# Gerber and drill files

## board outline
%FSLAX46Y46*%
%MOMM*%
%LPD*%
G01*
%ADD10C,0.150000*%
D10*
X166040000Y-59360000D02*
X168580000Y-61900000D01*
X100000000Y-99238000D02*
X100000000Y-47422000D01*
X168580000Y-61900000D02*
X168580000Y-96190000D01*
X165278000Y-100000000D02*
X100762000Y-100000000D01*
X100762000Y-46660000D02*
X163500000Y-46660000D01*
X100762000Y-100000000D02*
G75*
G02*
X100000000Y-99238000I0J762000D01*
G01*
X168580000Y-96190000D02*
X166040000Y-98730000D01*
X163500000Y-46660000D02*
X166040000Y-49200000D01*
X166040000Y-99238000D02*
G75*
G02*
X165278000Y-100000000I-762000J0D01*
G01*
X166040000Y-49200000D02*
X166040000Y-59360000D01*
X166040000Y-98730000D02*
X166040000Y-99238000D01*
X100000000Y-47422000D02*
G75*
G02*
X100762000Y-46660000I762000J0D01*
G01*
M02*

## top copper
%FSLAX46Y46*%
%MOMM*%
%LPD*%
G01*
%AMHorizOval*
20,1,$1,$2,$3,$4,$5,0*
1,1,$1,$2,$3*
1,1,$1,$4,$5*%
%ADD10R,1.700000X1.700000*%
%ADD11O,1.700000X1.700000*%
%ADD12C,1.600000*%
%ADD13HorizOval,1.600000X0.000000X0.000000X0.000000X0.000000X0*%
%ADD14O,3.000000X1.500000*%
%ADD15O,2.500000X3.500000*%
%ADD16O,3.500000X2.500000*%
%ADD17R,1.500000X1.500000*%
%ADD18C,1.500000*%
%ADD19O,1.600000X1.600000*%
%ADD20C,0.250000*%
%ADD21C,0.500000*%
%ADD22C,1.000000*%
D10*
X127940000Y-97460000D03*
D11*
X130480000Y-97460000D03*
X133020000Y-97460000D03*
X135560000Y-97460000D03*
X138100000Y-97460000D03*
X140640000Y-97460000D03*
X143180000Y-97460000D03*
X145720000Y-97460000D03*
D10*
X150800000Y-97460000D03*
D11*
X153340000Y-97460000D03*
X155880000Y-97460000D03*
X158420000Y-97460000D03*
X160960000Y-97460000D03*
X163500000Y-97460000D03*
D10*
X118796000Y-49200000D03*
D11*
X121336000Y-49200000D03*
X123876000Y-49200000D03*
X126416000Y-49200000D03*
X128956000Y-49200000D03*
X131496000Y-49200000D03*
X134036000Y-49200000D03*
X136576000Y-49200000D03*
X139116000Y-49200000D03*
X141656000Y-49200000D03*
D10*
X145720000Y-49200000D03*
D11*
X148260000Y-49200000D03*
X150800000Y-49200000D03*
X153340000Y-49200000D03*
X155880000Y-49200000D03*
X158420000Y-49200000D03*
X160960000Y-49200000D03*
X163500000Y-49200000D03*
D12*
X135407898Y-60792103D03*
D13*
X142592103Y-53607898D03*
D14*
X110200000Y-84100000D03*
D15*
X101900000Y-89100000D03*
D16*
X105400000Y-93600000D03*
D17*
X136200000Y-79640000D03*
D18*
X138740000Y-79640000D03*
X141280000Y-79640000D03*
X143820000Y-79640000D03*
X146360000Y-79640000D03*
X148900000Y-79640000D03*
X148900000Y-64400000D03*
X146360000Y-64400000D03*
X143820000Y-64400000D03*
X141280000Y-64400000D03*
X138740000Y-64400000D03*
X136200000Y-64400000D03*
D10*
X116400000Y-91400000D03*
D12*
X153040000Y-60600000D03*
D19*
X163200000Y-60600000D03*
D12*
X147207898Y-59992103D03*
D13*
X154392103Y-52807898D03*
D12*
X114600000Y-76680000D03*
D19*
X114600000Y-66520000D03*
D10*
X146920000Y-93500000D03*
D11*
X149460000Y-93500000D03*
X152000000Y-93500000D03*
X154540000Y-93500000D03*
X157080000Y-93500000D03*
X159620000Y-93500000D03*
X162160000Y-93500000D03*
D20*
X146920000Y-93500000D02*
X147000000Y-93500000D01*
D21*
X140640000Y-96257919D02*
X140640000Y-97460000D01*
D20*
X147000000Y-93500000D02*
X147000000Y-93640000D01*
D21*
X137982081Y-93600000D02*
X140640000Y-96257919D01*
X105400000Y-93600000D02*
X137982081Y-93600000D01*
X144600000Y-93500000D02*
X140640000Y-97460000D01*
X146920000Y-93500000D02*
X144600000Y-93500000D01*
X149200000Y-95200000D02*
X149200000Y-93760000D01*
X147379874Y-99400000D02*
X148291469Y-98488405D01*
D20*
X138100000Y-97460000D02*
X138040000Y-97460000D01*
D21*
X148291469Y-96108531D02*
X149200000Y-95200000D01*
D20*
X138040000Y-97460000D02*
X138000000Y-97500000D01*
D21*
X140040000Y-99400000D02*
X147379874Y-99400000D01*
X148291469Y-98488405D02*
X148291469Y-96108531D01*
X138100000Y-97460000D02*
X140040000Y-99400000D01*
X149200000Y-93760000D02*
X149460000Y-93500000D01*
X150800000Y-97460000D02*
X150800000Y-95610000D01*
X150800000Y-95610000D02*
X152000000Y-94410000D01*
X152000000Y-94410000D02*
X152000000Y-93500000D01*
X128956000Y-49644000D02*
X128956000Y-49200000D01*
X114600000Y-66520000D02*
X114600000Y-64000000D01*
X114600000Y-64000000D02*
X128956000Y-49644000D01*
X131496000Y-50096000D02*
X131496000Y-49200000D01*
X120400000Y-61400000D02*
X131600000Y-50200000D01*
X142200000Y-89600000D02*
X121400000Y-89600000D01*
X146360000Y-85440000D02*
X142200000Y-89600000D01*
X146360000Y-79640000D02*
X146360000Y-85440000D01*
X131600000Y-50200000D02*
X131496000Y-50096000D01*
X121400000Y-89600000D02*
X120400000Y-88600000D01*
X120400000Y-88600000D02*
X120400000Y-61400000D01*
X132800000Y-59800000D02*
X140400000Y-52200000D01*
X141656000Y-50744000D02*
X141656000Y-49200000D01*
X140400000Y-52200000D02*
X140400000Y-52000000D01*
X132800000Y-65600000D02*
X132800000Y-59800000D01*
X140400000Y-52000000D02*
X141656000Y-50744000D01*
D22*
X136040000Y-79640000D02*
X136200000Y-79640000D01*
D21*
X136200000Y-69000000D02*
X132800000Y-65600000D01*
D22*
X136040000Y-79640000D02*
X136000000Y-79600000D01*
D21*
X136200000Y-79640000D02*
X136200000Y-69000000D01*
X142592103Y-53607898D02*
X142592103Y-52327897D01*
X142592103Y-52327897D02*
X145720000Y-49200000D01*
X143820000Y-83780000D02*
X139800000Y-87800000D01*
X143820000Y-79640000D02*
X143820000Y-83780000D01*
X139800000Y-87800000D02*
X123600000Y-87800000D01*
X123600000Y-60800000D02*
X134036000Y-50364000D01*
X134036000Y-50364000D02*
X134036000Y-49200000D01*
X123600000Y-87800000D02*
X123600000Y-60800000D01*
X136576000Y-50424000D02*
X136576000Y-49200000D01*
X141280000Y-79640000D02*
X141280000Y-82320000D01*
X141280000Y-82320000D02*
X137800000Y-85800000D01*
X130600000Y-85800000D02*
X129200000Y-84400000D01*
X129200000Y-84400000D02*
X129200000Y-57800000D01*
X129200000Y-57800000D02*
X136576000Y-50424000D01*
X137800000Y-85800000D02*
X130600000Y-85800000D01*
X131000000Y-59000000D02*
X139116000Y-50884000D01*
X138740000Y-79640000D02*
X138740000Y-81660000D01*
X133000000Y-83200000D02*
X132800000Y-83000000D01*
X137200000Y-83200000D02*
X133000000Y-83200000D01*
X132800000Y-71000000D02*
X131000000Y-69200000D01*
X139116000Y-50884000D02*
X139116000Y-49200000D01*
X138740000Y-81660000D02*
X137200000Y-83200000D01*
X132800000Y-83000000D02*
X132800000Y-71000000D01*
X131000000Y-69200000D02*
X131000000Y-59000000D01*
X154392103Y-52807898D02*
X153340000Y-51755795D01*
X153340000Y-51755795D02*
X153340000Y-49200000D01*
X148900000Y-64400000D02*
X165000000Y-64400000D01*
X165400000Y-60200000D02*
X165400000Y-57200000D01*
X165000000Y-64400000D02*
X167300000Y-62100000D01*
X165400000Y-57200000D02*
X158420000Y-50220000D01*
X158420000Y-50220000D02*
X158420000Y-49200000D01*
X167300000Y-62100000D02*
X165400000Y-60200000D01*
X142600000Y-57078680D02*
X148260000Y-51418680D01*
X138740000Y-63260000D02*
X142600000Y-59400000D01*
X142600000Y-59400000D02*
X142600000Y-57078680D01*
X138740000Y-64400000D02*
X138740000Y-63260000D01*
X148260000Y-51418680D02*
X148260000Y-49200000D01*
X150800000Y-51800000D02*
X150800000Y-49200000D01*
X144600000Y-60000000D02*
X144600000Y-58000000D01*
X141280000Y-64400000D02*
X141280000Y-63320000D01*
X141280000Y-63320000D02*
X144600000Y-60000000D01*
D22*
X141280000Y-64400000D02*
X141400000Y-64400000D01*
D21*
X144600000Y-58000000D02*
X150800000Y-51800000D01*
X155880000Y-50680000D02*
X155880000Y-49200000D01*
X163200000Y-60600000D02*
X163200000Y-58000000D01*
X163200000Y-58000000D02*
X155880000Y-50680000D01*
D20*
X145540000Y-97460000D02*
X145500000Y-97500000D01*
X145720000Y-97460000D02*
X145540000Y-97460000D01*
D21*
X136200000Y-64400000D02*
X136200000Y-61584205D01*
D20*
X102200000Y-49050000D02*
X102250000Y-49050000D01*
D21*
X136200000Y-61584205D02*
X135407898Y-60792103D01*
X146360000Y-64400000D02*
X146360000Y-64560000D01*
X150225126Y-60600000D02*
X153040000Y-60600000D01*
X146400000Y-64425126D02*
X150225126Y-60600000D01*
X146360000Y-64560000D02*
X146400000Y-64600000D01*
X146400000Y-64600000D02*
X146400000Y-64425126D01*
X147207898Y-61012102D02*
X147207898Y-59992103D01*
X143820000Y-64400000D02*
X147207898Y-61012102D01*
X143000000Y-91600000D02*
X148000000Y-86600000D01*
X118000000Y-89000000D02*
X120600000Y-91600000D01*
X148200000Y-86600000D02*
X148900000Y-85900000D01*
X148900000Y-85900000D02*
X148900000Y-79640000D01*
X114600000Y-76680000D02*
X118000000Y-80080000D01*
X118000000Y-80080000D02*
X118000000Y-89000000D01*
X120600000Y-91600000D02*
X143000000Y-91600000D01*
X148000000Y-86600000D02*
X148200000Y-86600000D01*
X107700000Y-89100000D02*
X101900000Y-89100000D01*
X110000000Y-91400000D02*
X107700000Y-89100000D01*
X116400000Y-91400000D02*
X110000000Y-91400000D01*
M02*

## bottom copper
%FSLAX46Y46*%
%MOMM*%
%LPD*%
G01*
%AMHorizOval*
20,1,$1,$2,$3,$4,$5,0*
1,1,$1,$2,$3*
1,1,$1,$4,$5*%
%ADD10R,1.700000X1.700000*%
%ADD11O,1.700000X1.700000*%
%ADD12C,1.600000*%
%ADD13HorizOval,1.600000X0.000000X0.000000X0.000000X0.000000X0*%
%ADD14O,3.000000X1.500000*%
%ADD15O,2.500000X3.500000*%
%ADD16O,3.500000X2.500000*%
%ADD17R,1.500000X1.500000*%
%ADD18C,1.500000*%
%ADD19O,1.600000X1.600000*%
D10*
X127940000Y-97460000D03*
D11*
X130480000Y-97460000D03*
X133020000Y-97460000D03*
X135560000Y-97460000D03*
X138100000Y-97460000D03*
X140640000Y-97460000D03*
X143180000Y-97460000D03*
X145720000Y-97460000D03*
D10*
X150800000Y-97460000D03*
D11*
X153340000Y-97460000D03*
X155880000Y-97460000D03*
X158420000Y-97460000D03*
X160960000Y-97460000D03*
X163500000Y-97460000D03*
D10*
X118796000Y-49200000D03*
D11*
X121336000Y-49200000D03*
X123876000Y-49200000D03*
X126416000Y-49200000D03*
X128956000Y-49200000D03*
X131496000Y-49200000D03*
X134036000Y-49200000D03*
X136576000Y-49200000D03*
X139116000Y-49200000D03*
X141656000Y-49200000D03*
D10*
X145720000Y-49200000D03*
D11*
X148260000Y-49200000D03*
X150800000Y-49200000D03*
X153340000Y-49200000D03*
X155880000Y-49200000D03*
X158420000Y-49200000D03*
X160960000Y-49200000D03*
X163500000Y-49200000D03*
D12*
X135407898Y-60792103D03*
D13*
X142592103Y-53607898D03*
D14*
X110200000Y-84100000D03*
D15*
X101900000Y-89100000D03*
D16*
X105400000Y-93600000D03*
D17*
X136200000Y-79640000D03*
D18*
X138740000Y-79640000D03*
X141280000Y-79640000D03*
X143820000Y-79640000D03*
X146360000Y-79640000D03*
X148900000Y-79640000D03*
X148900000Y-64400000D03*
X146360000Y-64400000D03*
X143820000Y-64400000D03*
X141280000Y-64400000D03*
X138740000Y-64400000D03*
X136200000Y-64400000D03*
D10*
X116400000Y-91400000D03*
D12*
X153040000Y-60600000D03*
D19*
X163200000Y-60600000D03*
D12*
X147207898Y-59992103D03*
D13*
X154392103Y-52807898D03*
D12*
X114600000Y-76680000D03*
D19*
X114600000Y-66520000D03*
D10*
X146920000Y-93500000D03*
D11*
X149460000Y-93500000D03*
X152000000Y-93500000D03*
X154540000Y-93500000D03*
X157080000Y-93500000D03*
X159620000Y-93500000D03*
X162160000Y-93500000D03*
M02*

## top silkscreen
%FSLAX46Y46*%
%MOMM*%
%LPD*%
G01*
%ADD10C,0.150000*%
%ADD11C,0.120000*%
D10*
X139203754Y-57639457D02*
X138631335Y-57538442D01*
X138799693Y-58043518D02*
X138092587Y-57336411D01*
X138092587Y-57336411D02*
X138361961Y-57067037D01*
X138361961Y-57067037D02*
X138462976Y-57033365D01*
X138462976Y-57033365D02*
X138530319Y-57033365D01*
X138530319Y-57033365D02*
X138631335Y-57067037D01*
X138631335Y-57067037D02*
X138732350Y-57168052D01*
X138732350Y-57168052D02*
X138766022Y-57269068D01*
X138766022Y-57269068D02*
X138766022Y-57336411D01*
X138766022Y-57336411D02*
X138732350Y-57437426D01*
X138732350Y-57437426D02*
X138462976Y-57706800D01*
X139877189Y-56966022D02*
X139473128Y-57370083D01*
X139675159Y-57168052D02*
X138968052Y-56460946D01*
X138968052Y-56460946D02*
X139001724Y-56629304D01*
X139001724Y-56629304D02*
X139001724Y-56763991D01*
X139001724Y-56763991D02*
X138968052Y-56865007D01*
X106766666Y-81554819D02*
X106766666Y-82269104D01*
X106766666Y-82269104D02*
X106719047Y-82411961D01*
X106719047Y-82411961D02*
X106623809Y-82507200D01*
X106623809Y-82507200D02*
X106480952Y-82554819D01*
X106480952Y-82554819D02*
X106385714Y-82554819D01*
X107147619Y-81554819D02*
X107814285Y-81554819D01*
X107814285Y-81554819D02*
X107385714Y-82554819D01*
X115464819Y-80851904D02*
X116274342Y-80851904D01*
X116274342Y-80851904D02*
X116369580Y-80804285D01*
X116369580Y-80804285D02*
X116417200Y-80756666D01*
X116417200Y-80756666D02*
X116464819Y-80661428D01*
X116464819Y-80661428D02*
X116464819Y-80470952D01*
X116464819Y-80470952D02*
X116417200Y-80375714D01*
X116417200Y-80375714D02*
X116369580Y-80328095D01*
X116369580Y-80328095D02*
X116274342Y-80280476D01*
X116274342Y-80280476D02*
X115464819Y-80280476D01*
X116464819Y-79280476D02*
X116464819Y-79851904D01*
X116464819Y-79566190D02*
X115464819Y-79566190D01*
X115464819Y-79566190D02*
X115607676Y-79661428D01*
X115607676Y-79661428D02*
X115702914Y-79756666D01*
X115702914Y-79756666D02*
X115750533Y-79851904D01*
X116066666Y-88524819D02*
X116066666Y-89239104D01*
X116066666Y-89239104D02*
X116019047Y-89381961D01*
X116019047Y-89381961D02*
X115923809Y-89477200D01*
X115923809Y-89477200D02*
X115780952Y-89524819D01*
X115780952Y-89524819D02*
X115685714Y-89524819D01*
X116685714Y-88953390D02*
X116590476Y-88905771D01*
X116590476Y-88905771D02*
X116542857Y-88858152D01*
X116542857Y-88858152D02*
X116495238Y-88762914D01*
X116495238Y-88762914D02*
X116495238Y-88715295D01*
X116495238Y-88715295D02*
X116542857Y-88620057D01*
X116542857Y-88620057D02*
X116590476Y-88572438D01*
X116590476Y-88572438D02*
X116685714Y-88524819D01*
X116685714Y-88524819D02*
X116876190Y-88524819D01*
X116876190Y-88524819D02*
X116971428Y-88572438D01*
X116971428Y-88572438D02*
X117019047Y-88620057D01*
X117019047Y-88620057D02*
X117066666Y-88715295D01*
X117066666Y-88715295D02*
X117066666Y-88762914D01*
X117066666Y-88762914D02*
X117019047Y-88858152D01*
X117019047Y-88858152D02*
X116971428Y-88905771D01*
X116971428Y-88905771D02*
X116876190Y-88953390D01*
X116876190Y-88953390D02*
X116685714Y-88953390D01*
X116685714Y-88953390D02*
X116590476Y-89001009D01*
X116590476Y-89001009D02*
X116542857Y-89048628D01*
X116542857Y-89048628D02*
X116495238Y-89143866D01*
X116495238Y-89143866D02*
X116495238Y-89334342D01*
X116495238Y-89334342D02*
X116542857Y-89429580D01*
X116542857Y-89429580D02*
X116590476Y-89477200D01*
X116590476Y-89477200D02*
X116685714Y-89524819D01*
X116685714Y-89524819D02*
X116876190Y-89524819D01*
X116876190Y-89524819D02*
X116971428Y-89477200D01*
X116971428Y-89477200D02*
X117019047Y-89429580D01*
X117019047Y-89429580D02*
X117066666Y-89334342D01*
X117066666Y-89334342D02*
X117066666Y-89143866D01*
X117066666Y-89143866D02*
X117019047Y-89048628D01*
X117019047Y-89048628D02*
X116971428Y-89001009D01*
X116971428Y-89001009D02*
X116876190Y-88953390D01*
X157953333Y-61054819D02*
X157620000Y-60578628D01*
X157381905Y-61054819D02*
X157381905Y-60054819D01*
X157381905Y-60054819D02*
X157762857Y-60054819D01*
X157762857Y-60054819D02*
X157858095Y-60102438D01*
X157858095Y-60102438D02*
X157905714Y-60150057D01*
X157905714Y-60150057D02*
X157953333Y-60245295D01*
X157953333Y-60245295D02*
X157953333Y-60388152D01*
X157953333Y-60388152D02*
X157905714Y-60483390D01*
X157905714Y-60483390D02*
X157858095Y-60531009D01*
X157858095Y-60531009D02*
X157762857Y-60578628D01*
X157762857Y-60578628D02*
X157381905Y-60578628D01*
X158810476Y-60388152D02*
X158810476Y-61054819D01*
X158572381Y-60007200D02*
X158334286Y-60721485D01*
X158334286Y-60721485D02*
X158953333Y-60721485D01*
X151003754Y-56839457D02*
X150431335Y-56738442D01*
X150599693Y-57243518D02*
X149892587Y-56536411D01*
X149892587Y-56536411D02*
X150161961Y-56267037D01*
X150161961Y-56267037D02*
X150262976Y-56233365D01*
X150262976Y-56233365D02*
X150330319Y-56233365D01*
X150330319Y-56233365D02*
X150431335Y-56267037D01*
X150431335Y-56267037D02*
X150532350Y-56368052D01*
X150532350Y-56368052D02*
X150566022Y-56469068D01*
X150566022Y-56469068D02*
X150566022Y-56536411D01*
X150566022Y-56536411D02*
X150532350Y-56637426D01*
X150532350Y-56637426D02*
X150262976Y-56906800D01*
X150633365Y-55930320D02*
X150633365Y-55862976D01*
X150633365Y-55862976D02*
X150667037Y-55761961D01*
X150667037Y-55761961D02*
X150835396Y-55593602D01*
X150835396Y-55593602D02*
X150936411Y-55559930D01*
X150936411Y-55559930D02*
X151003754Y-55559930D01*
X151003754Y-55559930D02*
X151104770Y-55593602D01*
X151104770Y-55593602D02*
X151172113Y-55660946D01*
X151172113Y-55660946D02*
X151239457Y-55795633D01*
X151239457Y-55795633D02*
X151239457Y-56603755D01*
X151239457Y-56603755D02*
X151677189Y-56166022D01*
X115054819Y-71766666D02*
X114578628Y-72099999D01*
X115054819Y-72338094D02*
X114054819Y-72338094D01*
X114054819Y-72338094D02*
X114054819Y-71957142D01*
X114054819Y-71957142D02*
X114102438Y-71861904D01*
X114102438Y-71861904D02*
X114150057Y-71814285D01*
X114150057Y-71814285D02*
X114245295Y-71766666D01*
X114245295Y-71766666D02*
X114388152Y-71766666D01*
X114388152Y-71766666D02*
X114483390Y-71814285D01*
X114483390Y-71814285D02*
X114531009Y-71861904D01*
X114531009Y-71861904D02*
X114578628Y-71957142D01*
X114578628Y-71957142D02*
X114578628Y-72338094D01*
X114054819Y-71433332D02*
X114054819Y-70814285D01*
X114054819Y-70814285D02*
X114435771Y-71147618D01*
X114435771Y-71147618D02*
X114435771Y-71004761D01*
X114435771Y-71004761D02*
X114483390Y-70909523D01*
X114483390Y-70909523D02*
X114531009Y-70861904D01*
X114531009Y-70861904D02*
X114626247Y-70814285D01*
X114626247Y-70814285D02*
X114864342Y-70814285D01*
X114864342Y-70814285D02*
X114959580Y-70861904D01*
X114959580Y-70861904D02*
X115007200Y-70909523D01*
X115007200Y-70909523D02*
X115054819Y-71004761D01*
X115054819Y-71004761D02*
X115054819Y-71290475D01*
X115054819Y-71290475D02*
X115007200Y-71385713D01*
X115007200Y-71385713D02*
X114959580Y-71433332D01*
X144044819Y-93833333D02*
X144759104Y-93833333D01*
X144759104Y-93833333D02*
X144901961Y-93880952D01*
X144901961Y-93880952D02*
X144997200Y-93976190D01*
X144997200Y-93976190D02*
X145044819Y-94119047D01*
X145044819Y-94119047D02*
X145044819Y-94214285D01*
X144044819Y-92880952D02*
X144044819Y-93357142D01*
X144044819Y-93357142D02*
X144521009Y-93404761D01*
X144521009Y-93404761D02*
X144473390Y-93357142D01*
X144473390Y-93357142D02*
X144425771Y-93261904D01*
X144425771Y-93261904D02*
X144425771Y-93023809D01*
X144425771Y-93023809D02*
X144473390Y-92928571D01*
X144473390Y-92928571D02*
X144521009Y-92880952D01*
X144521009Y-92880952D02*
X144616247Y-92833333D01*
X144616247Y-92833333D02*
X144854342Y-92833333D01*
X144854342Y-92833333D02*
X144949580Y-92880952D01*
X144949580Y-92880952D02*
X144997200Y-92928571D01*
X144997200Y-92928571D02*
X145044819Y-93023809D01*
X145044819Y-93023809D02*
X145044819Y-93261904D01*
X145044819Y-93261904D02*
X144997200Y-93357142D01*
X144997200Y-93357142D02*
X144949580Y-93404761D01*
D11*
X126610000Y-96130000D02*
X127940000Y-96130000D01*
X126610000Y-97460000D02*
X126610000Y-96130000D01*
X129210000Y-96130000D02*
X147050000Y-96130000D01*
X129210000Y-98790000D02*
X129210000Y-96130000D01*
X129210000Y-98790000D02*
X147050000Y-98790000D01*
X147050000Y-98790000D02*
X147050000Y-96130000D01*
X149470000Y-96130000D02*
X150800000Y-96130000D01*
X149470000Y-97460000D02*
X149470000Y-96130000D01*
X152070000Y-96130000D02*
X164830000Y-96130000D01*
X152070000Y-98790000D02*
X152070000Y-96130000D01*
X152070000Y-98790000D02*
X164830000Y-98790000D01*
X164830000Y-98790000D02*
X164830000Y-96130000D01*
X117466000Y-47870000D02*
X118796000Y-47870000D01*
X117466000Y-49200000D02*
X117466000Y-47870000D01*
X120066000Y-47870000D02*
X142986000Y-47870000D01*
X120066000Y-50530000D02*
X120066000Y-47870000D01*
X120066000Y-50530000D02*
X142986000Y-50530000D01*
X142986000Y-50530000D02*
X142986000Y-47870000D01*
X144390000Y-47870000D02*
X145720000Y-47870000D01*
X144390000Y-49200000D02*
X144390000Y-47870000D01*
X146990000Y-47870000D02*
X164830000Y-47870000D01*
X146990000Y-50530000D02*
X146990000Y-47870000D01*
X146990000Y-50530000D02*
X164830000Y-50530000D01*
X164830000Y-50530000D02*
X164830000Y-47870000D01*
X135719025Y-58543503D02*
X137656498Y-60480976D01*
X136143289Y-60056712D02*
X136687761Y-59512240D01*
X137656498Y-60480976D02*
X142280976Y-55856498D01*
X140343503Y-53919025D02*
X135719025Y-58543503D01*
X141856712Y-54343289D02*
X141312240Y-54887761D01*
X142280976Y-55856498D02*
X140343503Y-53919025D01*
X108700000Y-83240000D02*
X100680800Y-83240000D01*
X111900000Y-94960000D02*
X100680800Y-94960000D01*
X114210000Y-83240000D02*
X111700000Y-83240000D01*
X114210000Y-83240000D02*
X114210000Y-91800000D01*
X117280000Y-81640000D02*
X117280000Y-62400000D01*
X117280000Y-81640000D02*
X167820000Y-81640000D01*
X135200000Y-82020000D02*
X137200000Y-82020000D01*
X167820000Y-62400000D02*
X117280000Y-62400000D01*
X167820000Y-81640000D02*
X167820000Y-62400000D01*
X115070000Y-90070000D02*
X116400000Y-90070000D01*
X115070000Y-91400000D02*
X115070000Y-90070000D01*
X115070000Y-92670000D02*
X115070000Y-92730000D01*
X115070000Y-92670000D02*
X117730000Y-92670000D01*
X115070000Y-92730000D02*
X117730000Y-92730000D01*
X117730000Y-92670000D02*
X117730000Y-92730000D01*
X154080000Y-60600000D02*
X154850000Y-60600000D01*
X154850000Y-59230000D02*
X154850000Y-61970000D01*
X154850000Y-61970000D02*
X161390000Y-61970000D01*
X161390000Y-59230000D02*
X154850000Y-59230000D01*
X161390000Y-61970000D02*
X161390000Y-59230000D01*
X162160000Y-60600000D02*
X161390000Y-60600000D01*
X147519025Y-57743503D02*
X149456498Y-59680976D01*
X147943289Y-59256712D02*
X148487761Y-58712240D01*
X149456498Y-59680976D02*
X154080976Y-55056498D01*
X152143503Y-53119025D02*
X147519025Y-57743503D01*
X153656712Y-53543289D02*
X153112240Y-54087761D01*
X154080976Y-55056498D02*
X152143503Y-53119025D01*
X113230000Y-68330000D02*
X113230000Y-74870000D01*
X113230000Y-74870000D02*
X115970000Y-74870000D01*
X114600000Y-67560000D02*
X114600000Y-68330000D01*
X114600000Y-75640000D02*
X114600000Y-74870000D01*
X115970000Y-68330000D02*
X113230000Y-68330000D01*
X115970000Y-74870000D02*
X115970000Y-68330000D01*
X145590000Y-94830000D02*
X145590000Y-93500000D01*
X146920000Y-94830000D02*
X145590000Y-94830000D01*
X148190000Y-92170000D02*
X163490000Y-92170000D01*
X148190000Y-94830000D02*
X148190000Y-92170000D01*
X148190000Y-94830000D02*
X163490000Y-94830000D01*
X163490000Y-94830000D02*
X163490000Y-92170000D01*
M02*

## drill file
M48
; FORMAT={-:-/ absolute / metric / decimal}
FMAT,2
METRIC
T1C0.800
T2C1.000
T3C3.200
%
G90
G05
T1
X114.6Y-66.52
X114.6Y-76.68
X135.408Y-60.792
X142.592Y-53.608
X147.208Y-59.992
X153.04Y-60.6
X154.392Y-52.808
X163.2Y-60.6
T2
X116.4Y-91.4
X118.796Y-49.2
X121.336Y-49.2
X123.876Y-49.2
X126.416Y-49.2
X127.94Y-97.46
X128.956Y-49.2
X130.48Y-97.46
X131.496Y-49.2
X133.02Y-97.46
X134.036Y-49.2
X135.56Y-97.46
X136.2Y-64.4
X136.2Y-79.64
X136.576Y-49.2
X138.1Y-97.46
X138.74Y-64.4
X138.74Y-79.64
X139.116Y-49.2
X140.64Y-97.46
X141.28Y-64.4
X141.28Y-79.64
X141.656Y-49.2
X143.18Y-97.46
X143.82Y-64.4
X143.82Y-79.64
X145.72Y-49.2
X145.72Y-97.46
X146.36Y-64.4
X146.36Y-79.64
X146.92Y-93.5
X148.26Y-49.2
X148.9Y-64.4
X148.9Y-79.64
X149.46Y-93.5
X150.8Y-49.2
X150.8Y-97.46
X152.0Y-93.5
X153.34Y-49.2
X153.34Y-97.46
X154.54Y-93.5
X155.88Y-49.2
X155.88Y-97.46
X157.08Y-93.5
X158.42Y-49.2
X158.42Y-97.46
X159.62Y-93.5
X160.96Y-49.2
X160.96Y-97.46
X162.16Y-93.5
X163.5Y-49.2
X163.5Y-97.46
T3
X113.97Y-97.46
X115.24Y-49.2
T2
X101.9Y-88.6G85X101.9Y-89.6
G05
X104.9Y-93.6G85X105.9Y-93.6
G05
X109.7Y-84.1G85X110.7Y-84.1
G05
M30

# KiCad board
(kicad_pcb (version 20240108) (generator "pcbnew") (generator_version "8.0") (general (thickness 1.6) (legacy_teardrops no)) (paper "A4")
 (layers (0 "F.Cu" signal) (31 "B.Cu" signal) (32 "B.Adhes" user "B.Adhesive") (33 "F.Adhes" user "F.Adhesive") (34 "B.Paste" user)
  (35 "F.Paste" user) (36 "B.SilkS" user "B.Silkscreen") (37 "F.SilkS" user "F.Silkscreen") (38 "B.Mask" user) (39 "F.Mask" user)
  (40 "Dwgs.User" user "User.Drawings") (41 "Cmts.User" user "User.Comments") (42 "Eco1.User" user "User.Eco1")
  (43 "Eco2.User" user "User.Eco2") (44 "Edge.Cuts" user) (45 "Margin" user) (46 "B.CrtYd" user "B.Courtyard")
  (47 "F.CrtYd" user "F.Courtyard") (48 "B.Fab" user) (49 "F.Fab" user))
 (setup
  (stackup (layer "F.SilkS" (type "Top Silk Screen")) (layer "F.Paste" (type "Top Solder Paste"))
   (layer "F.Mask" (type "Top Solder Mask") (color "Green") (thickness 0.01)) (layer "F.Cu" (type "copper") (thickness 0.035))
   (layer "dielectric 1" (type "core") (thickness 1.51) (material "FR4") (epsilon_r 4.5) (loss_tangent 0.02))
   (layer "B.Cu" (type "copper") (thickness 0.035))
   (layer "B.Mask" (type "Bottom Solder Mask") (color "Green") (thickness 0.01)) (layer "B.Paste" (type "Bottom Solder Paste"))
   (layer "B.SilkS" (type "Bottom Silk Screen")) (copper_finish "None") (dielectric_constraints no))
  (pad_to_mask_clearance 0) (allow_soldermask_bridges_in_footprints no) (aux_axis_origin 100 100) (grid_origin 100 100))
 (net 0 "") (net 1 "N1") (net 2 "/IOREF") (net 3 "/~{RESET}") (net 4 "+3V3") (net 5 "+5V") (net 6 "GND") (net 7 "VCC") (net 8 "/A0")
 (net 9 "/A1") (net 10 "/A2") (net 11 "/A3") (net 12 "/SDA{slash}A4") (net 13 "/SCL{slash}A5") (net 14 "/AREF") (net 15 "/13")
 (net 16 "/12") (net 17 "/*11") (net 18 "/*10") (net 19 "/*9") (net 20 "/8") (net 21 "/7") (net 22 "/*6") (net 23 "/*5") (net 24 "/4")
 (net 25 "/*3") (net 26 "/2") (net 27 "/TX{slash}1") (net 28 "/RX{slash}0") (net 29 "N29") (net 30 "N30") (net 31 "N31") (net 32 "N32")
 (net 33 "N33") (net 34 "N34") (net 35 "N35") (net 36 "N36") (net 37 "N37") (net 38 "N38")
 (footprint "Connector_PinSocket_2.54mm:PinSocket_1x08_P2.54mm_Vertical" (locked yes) (layer "F.Cu") (at 127.94 97.46 90)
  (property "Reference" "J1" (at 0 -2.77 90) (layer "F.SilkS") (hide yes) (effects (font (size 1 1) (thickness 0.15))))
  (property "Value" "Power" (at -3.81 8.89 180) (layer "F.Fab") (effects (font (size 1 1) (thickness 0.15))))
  (fp_line (start 1.33 -1.33) (end 1.33 0) (stroke (width 0.12) (type solid)) (layer "F.SilkS"))
  (fp_line (start 0 -1.33) (end 1.33 -1.33) (stroke (width 0.12) (type solid)) (layer "F.SilkS"))
  (fp_line (start 1.33 1.27) (end 1.33 19.11) (stroke (width 0.12) (type solid)) (layer "F.SilkS"))
  (fp_line (start -1.33 1.27) (end 1.33 1.27) (stroke (width 0.12) (type solid)) (layer "F.SilkS"))
  (fp_line (start -1.33 1.27) (end -1.33 19.11) (stroke (width 0.12) (type solid)) (layer "F.SilkS"))
  (fp_line (start -1.33 19.11) (end 1.33 19.11) (stroke (width 0.12) (type solid)) (layer "F.SilkS"))
  (pad "1" thru_hole rect (at 0 0 90) (size 1.7 1.7) (drill 1) (layers "*.Cu" "*.Mask") (remove_unused_layers no) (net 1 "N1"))
  (pad "2" thru_hole oval (at 0 2.54 90) (size 1.7 1.7) (drill 1) (layers "*.Cu" "*.Mask") (remove_unused_layers no) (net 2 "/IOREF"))
  (pad "3" thru_hole oval (at 0 5.08 90) (size 1.7 1.7) (drill 1) (layers "*.Cu" "*.Mask") (remove_unused_layers no) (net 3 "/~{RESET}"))
  (pad "4" thru_hole oval (at 0 7.62 90) (size 1.7 1.7) (drill 1) (layers "*.Cu" "*.Mask") (remove_unused_layers no) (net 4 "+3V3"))
  (pad "5" thru_hole oval (at 0 10.16 90) (size 1.7 1.7) (drill 1) (layers "*.Cu" "*.Mask") (remove_unused_layers no) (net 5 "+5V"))
  (pad "6" thru_hole oval (at 0 12.7 90) (size 1.7 1.7) (drill 1) (layers "*.Cu" "*.Mask") (remove_unused_layers no) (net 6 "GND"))
  (pad "7" thru_hole oval (at 0 15.24 90) (size 1.7 1.7) (drill 1) (layers "*.Cu" "*.Mask") (remove_unused_layers no) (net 6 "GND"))
  (pad "8" thru_hole oval (at 0 17.78 90) (size 1.7 1.7) (drill 1) (layers "*.Cu" "*.Mask") (remove_unused_layers no) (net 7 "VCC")))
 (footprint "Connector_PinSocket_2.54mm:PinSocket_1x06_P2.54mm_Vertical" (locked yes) (layer "F.Cu") (at 150.8 97.46 90)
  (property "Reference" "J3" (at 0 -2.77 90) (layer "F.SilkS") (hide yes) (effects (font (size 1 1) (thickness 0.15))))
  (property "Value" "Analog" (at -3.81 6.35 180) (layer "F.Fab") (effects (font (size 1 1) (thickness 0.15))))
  (fp_line (start 1.33 -1.33) (end 1.33 0) (stroke (width 0.12) (type solid)) (layer "F.SilkS"))
  (fp_line (start 0 -1.33) (end 1.33 -1.33) (stroke (width 0.12) (type solid)) (layer "F.SilkS"))
  (fp_line (start 1.33 1.27) (end 1.33 14.03) (stroke (width 0.12) (type solid)) (layer "F.SilkS"))
  (fp_line (start -1.33 1.27) (end 1.33 1.27) (stroke (width 0.12) (type solid)) (layer "F.SilkS"))
  (fp_line (start -1.33 1.27) (end -1.33 14.03) (stroke (width 0.12) (type solid)) (layer "F.SilkS"))
  (fp_line (start -1.33 14.03) (end 1.33 14.03) (stroke (width 0.12) (type solid)) (layer "F.SilkS"))
  (pad "1" thru_hole rect (at 0 0 90) (size 1.7 1.7) (drill 1) (layers "*.Cu" "*.Mask") (remove_unused_layers no) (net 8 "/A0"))
  (pad "2" thru_hole oval (at 0 2.54 90) (size 1.7 1.7) (drill 1) (layers "*.Cu" "*.Mask") (remove_unused_layers no) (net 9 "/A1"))
  (pad "3" thru_hole oval (at 0 5.08 90) (size 1.7 1.7) (drill 1) (layers "*.Cu" "*.Mask") (remove_unused_layers no) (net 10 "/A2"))
  (pad "4" thru_hole oval (at 0 7.62 90) (size 1.7 1.7) (drill 1) (layers "*.Cu" "*.Mask") (remove_unused_layers no) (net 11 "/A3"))
  (pad "5" thru_hole oval (at 0 10.16 90) (size 1.7 1.7) (drill 1) (layers "*.Cu" "*.Mask") (remove_unused_layers no)
   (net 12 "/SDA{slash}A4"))
  (pad "6" thru_hole oval (at 0 12.7 90) (size 1.7 1.7) (drill 1) (layers "*.Cu" "*.Mask") (remove_unused_layers no)
   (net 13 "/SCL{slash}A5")))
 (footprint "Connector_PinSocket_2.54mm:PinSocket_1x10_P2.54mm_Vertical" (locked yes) (layer "F.Cu") (at 118.796 49.2 90)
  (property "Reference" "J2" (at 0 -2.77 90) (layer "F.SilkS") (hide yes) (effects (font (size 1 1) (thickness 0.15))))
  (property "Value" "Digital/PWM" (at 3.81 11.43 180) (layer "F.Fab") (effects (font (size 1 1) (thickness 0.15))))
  (fp_line (start 1.33 -1.33) (end 1.33 0) (stroke (width 0.12) (type solid)) (layer "F.SilkS"))
  (fp_line (start 0 -1.33) (end 1.33 -1.33) (stroke (width 0.12) (type solid)) (layer "F.SilkS"))
  (fp_line (start 1.33 1.27) (end 1.33 24.19) (stroke (width 0.12) (type solid)) (layer "F.SilkS"))
  (fp_line (start -1.33 1.27) (end 1.33 1.27) (stroke (width 0.12) (type solid)) (layer "F.SilkS"))
  (fp_line (start -1.33 1.27) (end -1.33 24.19) (stroke (width 0.12) (type solid)) (layer "F.SilkS"))
  (fp_line (start -1.33 24.19) (end 1.33 24.19) (stroke (width 0.12) (type solid)) (layer "F.SilkS"))
  (pad "1" thru_hole rect (at 0 0 90) (size 1.7 1.7) (drill 1) (layers "*.Cu" "*.Mask") (remove_unused_layers no) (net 13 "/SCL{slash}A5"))
  (pad "2" thru_hole oval (at 0 2.54 90) (size 1.7 1.7) (drill 1) (layers "*.Cu" "*.Mask") (remove_unused_layers no)
   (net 12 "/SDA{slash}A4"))
  (pad "3" thru_hole oval (at 0 5.08 90) (size 1.7 1.7) (drill 1) (layers "*.Cu" "*.Mask") (remove_unused_layers no) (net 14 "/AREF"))
  (pad "4" thru_hole oval (at 0 7.62 90) (size 1.7 1.7) (drill 1) (layers "*.Cu" "*.Mask") (remove_unused_layers no) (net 6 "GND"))
  (pad "5" thru_hole oval (at 0 10.16 90) (size 1.7 1.7) (drill 1) (layers "*.Cu" "*.Mask") (remove_unused_layers no) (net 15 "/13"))
  (pad "6" thru_hole oval (at 0 12.7 90) (size 1.7 1.7) (drill 1) (layers "*.Cu" "*.Mask") (remove_unused_layers no) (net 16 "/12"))
  (pad "7" thru_hole oval (at 0 15.24 90) (size 1.7 1.7) (drill 1) (layers "*.Cu" "*.Mask") (remove_unused_layers no) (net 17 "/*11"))
  (pad "8" thru_hole oval (at 0 17.78 90) (size 1.7 1.7) (drill 1) (layers "*.Cu" "*.Mask") (remove_unused_layers no) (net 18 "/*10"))
  (pad "9" thru_hole oval (at 0 20.32 90) (size 1.7 1.7) (drill 1) (layers "*.Cu" "*.Mask") (remove_unused_layers no) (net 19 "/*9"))
  (pad "10" thru_hole oval (at 0 22.86 90) (size 1.7 1.7) (drill 1) (layers "*.Cu" "*.Mask") (remove_unused_layers no) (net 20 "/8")))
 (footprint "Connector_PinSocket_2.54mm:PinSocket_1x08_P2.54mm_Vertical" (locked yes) (layer "F.Cu") (at 145.72 49.2 90)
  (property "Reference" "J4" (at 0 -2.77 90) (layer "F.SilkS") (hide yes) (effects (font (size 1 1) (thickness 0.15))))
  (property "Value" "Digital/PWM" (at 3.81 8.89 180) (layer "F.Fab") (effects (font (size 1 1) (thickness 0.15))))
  (fp_line (start 1.33 -1.33) (end 1.33 0) (stroke (width 0.12) (type solid)) (layer "F.SilkS"))
  (fp_line (start 0 -1.33) (end 1.33 -1.33) (stroke (width 0.12) (type solid)) (layer "F.SilkS"))
  (fp_line (start 1.33 1.27) (end 1.33 19.11) (stroke (width 0.12) (type solid)) (layer "F.SilkS"))
  (fp_line (start -1.33 1.27) (end 1.33 1.27) (stroke (width 0.12) (type solid)) (layer "F.SilkS"))
  (fp_line (start -1.33 1.27) (end -1.33 19.11) (stroke (width 0.12) (type solid)) (layer "F.SilkS"))
  (fp_line (start -1.33 19.11) (end 1.33 19.11) (stroke (width 0.12) (type solid)) (layer "F.SilkS"))
  (pad "1" thru_hole rect (at 0 0 90) (size 1.7 1.7) (drill 1) (layers "*.Cu" "*.Mask") (remove_unused_layers no) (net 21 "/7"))
  (pad "2" thru_hole oval (at 0 2.54 90) (size 1.7 1.7) (drill 1) (layers "*.Cu" "*.Mask") (remove_unused_layers no) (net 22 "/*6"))
  (pad "3" thru_hole oval (at 0 5.08 90) (size 1.7 1.7) (drill 1) (layers "*.Cu" "*.Mask") (remove_unused_layers no) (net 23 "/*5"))
  (pad "4" thru_hole oval (at 0 7.62 90) (size 1.7 1.7) (drill 1) (layers "*.Cu" "*.Mask") (remove_unused_layers no) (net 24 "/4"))
  (pad "5" thru_hole oval (at 0 10.16 90) (size 1.7 1.7) (drill 1) (layers "*.Cu" "*.Mask") (remove_unused_layers no) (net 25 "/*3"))
  (pad "6" thru_hole oval (at 0 12.7 90) (size 1.7 1.7) (drill 1) (layers "*.Cu" "*.Mask") (remove_unused_layers no) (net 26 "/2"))
  (pad "7" thru_hole oval (at 0 15.24 90) (size 1.7 1.7) (drill 1) (layers "*.Cu" "*.Mask") (remove_unused_layers no) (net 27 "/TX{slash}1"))
  (pad "8" thru_hole oval (at 0 17.78 90) (size 1.7 1.7) (drill 1) (layers "*.Cu" "*.Mask") (remove_unused_layers no) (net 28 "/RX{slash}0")))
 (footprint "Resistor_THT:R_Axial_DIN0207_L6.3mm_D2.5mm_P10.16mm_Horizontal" (layer "F.Cu") (at 135.407898 60.792103 45)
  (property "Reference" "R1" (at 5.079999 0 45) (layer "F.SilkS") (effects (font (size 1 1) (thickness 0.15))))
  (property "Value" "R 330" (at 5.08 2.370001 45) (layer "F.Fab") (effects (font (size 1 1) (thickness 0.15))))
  (fp_line (start 1.81 -1.37) (end 1.81 1.37) (stroke (width 0.12) (type solid)) (layer "F.SilkS"))
  (fp_line (start 1.04 0) (end 1.81 0) (stroke (width 0.12) (type solid)) (layer "F.SilkS"))
  (fp_line (start 1.81 1.37) (end 8.35 1.37) (stroke (width 0.12) (type solid)) (layer "F.SilkS"))
  (fp_line (start 8.35 -1.37) (end 1.81 -1.37) (stroke (width 0.12) (type solid)) (layer "F.SilkS"))
  (fp_line (start 9.12 0) (end 8.350001 0) (stroke (width 0.12) (type solid)) (layer "F.SilkS"))
  (fp_line (start 8.35 1.37) (end 8.35 -1.37) (stroke (width 0.12) (type solid)) (layer "F.SilkS"))
  (pad "1" thru_hole circle (at 0 0 45) (size 1.6 1.6) (drill 0.8) (layers "*.Cu" "*.Mask") (remove_unused_layers no) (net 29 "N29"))
  (pad "2" thru_hole oval (at 10.16 0 45) (size 1.6 1.6) (drill 0.8) (layers "*.Cu" "*.Mask") (remove_unused_layers no) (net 21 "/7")))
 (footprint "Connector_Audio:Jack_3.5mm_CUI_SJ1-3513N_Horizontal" (layer "F.Cu") (at 101.9 89.1)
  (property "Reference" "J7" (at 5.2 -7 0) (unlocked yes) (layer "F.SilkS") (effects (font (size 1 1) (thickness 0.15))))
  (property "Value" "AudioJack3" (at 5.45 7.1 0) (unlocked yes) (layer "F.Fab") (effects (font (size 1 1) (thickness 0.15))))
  (fp_line (start 6.8 -5.86) (end -1.2192 -5.86) (stroke (width 0.12) (type solid)) (layer "F.SilkS"))
  (fp_line (start 10 5.86) (end -1.2192 5.86) (stroke (width 0.12) (type solid)) (layer "F.SilkS"))
  (fp_line (start 12.31 -5.86) (end 9.8 -5.86) (stroke (width 0.12) (type solid)) (layer "F.SilkS"))
  (fp_line (start 12.31 -5.86) (end 12.31 2.7) (stroke (width 0.12) (type solid)) (layer "F.SilkS"))
  (pad "R" thru_hole oval (at 8.3 -5) (size 3 1.5) (drill oval 2 1) (layers "*.Cu" "*.Mask") (remove_unused_layers no) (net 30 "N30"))
  (pad "S" thru_hole oval (at 0 0 270) (size 3.5 2.5) (drill oval 2 1) (layers "*.Cu" "*.Mask") (remove_unused_layers no) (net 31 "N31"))
  (pad "T" thru_hole oval (at 3.5 4.5) (size 3.5 2.5) (drill oval 2 1) (layers "*.Cu" "*.Mask") (remove_unused_layers no) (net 6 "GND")))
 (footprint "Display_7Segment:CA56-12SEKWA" (layer "F.Cu") (at 136.2 79.64 90)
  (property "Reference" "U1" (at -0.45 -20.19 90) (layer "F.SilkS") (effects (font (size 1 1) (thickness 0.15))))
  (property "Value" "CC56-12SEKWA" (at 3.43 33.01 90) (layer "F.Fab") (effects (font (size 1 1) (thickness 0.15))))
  (fp_line (start -2 -18.92) (end 17.24 -18.92) (stroke (width 0.12) (type solid)) (layer "F.SilkS"))
  (fp_line (start -2 -18.92) (end -2 31.62) (stroke (width 0.12) (type solid)) (layer "F.SilkS"))
  (fp_line (start -2.38 -1) (end -2.38 1) (stroke (width 0.12) (type solid)) (layer "F.SilkS"))
  (fp_line (start 17.24 31.62) (end 17.24 -18.92) (stroke (width 0.12) (type solid)) (layer "F.SilkS"))
  (fp_line (start -2 31.62) (end 17.24 31.62) (stroke (width 0.12) (type solid)) (layer "F.SilkS"))
  (pad "1" thru_hole rect (at 0 0 90) (size 1.5 1.5) (drill 1) (layers "*.Cu" "*.Mask") (remove_unused_layers no) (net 20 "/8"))
  (pad "2" thru_hole circle (at 0 2.54 90) (size 1.5 1.5) (drill 1) (layers "*.Cu" "*.Mask") (remove_unused_layers no) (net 19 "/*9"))
  (pad "3" thru_hole circle (at 0 5.08 90) (size 1.5 1.5) (drill 1) (layers "*.Cu" "*.Mask") (remove_unused_layers no) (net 18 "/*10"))
  (pad "4" thru_hole circle (at 0 7.62 90) (size 1.5 1.5) (drill 1) (layers "*.Cu" "*.Mask") (remove_unused_layers no) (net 17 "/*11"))
  (pad "5" thru_hole circle (at 0 10.16 90) (size 1.5 1.5) (drill 1) (layers "*.Cu" "*.Mask") (remove_unused_layers no) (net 16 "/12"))
  (pad "6" thru_hole circle (at 0 12.7 90) (size 1.5 1.5) (drill 1) (layers "*.Cu" "*.Mask") (remove_unused_layers no) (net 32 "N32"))
  (pad "7" thru_hole circle (at 15.24 12.7 90) (size 1.5 1.5) (drill 1) (layers "*.Cu" "*.Mask") (remove_unused_layers no) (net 26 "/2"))
  (pad "8" thru_hole circle (at 15.24 10.16 90) (size 1.5 1.5) (drill 1) (layers "*.Cu" "*.Mask") (remove_unused_layers no) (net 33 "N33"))
  (pad "9" thru_hole circle (at 15.24 7.62 90) (size 1.5 1.5) (drill 1) (layers "*.Cu" "*.Mask") (remove_unused_layers no) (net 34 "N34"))
  (pad "10" thru_hole circle (at 15.24 5.08 90) (size 1.5 1.5) (drill 1) (layers "*.Cu" "*.Mask") (remove_unused_layers no) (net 23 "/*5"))
  (pad "11" thru_hole circle (at 15.24 2.54 90) (size 1.5 1.5) (drill 1) (layers "*.Cu" "*.Mask") (remove_unused_layers no) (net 22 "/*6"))
  (pad "12" thru_hole circle (at 15.24 0 90) (size 1.5 1.5) (drill 1) (layers "*.Cu" "*.Mask") (remove_unused_layers no) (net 29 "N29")))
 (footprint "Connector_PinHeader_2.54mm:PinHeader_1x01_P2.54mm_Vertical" (layer "F.Cu") (at 116.4 91.4)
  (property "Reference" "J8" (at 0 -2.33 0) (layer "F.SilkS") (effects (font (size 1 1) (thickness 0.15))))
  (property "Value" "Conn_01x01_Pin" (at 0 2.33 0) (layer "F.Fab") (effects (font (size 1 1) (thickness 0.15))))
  (fp_line (start -1.33 -1.33) (end 0 -1.33) (stroke (width 0.12) (type solid)) (layer "F.SilkS"))
  (fp_line (start -1.33 0) (end -1.33 -1.33) (stroke (width 0.12) (type solid)) (layer "F.SilkS"))
  (fp_line (start -1.33 1.27) (end -1.33 1.33) (stroke (width 0.12) (type solid)) (layer "F.SilkS"))
  (fp_line (start -1.33 1.27) (end 1.33 1.27) (stroke (width 0.12) (type solid)) (layer "F.SilkS"))
  (fp_line (start -1.33 1.33) (end 1.33 1.33) (stroke (width 0.12) (type solid)) (layer "F.SilkS"))
  (fp_line (start 1.33 1.27) (end 1.33 1.33) (stroke (width 0.12) (type solid)) (layer "F.SilkS"))
  (pad "1" thru_hole rect (at 0 0) (size 1.7 1.7) (drill 1) (layers "*.Cu" "*.Mask") (remove_unused_layers no) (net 31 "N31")))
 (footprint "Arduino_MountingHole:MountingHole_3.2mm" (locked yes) (layer "F.Cu") (at 115.24 49.2)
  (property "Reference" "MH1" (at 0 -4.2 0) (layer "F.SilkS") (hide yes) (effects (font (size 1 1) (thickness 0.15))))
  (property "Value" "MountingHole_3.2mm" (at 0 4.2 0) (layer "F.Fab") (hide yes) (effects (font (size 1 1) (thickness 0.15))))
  (pad "" np_thru_hole circle (at 0 0) (size 3.2 3.2) (drill 3.2) (layers "*.Cu" "*.Mask")))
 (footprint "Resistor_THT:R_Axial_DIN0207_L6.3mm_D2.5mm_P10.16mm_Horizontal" (layer "F.Cu") (at 153.04 60.6)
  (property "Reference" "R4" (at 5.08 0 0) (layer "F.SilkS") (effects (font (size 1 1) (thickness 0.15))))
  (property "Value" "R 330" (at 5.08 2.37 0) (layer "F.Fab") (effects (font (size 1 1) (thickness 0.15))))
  (fp_line (start 1.04 0) (end 1.81 0) (stroke (width 0.12) (type solid)) (layer "F.SilkS"))
  (fp_line (start 1.81 -1.37) (end 1.81 1.37) (stroke (width 0.12) (type solid)) (layer "F.SilkS"))
  (fp_line (start 1.81 1.37) (end 8.35 1.37) (stroke (width 0.12) (type solid)) (layer "F.SilkS"))
  (fp_line (start 8.35 -1.37) (end 1.81 -1.37) (stroke (width 0.12) (type solid)) (layer "F.SilkS"))
  (fp_line (start 8.35 1.37) (end 8.35 -1.37) (stroke (width 0.12) (type solid)) (layer "F.SilkS"))
  (fp_line (start 9.12 0) (end 8.35 0) (stroke (width 0.12) (type solid)) (layer "F.SilkS"))
  (pad "1" thru_hole circle (at 0 0) (size 1.6 1.6) (drill 0.8) (layers "*.Cu" "*.Mask") (remove_unused_layers no) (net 33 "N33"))
  (pad "2" thru_hole oval (at 10.16 0) (size 1.6 1.6) (drill 0.8) (layers "*.Cu" "*.Mask") (remove_unused_layers no) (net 25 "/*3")))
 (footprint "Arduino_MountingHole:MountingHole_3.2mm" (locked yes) (layer "F.Cu") (at 113.97 97.46)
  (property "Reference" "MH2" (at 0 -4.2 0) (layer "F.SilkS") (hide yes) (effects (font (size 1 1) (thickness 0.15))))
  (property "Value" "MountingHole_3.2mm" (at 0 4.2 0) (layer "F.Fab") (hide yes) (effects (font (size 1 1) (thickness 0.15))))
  (pad "" np_thru_hole circle (at 0 0) (size 3.2 3.2) (drill 3.2) (layers "*.Cu" "*.Mask")))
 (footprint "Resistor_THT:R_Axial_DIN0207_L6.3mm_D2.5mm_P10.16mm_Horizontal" (layer "F.Cu") (at 147.207898 59.992103 45)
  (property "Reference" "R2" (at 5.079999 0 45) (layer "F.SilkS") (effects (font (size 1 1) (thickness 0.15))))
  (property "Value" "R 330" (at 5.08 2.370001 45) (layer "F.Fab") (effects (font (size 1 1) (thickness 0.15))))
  (fp_line (start 1.81 -1.37) (end 1.81 1.37) (stroke (width 0.12) (type solid)) (layer "F.SilkS"))
  (fp_line (start 1.04 0) (end 1.81 0) (stroke (width 0.12) (type solid)) (layer "F.SilkS"))
  (fp_line (start 1.81 1.37) (end 8.35 1.37) (stroke (width 0.12) (type solid)) (layer "F.SilkS"))
  (fp_line (start 8.35 -1.37) (end 1.81 -1.37) (stroke (width 0.12) (type solid)) (layer "F.SilkS"))
  (fp_line (start 9.12 0) (end 8.350001 0) (stroke (width 0.12) (type solid)) (layer "F.SilkS"))
  (fp_line (start 8.35 1.37) (end 8.35 -1.37) (stroke (width 0.12) (type solid)) (layer "F.SilkS"))
  (pad "1" thru_hole circle (at 0 0 45) (size 1.6 1.6) (drill 0.8) (layers "*.Cu" "*.Mask") (remove_unused_layers no) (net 34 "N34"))
  (pad "2" thru_hole oval (at 10.16 0 45) (size 1.6 1.6) (drill 0.8) (layers "*.Cu" "*.Mask") (remove_unused_layers no) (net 24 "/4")))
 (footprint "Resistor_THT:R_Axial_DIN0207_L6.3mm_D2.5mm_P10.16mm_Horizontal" (layer "F.Cu") (at 114.6 76.68 90)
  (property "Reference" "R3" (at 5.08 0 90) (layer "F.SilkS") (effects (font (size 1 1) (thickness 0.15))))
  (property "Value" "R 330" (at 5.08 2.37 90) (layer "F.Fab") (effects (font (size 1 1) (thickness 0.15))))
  (fp_line (start 8.35 -1.37) (end 1.81 -1.37) (stroke (width 0.12) (type solid)) (layer "F.SilkS"))
  (fp_line (start 1.81 -1.37) (end 1.81 1.37) (stroke (width 0.12) (type solid)) (layer "F.SilkS"))
  (fp_line (start 9.12 0) (end 8.35 0) (stroke (width 0.12) (type solid)) (layer "F.SilkS"))
  (fp_line (start 1.04 0) (end 1.81 0) (stroke (width 0.12) (type solid)) (layer "F.SilkS"))
  (fp_line (start 8.35 1.37) (end 8.35 -1.37) (stroke (width 0.12) (type solid)) (layer "F.SilkS"))
  (fp_line (start 1.81 1.37) (end 8.35 1.37) (stroke (width 0.12) (type solid)) (layer "F.SilkS"))
  (pad "1" thru_hole circle (at 0 0 90) (size 1.6 1.6) (drill 0.8) (layers "*.Cu" "*.Mask") (remove_unused_layers no) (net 32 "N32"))
  (pad "2" thru_hole oval (at 10.16 0 90) (size 1.6 1.6) (drill 0.8) (layers "*.Cu" "*.Mask") (remove_unused_layers no) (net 15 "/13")))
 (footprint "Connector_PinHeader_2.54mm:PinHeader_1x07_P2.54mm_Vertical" (layer "F.Cu") (at 146.92 93.5 90)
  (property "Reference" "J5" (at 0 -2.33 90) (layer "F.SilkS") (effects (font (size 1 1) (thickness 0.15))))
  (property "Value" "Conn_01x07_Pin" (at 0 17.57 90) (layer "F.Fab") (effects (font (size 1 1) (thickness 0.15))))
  (fp_line (start -1.33 -1.33) (end 0 -1.33) (stroke (width 0.12) (type solid)) (layer "F.SilkS"))
  (fp_line (start -1.33 0) (end -1.33 -1.33) (stroke (width 0.12) (type solid)) (layer "F.SilkS"))
  (fp_line (start 1.33 1.27) (end 1.33 16.57) (stroke (width 0.12) (type solid)) (layer "F.SilkS"))
  (fp_line (start -1.33 1.27) (end 1.33 1.27) (stroke (width 0.12) (type solid)) (layer "F.SilkS"))
  (fp_line (start -1.33 1.27) (end -1.33 16.57) (stroke (width 0.12) (type solid)) (layer "F.SilkS"))
  (fp_line (start -1.33 16.57) (end 1.33 16.57) (stroke (width 0.12) (type solid)) (layer "F.SilkS"))
  (pad "1" thru_hole rect (at 0 0 90) (size 1.7 1.7) (drill 1) (layers "*.Cu" "*.Mask") (remove_unused_layers no) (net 6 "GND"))
  (pad "2" thru_hole oval (at 0 2.54 90) (size 1.7 1.7) (drill 1) (layers "*.Cu" "*.Mask") (remove_unused_layers no) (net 5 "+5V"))
  (pad "3" thru_hole oval (at 0 5.08 90) (size 1.7 1.7) (drill 1) (layers "*.Cu" "*.Mask") (remove_unused_layers no) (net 8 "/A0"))
  (pad "4" thru_hole oval (at 0 7.62 90) (size 1.7 1.7) (drill 1) (layers "*.Cu" "*.Mask") (remove_unused_layers no) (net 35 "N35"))
  (pad "5" thru_hole oval (at 0 10.16 90) (size 1.7 1.7) (drill 1) (layers "*.Cu" "*.Mask") (remove_unused_layers no) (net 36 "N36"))
  (pad "6" thru_hole oval (at 0 12.7 90) (size 1.7 1.7) (drill 1) (layers "*.Cu" "*.Mask") (remove_unused_layers no) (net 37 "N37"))
  (pad "7" thru_hole oval (at 0 15.24 90) (size 1.7 1.7) (drill 1) (layers "*.Cu" "*.Mask") (remove_unused_layers no) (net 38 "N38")))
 (gr_line (start 166.04 59.36) (end 168.58 61.9) (stroke (width 0.15) (type solid)) (layer "Edge.Cuts"))
 (gr_line (start 100 99.238) (end 100 47.422) (stroke (width 0.15) (type solid)) (layer "Edge.Cuts"))
 (gr_line (start 168.58 61.9) (end 168.58 96.19) (stroke (width 0.15) (type solid)) (layer "Edge.Cuts"))
 (gr_line (start 165.278 100) (end 100.762 100) (stroke (width 0.15) (type solid)) (layer "Edge.Cuts"))
 (gr_line (start 100.762 46.66) (end 163.5 46.66) (stroke (width 0.15) (type solid)) (layer "Edge.Cuts"))
 (gr_arc (start 100.762 100) (mid 100.223185 99.776815) (end 100 99.238) (stroke (width 0.15) (type solid)) (layer "Edge.Cuts"))
 (gr_line (start 168.58 96.19) (end 166.04 98.73) (stroke (width 0.15) (type solid)) (layer "Edge.Cuts"))
 (gr_line (start 163.5 46.66) (end 166.04 49.2) (stroke (width 0.15) (type solid)) (layer "Edge.Cuts"))
 (gr_arc (start 166.04 99.238) (mid 165.816815 99.776815) (end 165.278 100) (stroke (width 0.15) (type solid)) (layer "Edge.Cuts"))
 (gr_line (start 166.04 49.2) (end 166.04 59.36) (stroke (width 0.15) (type solid)) (layer "Edge.Cuts"))
 (gr_line (start 166.04 98.73) (end 166.04 99.238) (stroke (width 0.15) (type solid)) (layer "Edge.Cuts"))
 (gr_arc (start 100 47.422) (mid 100.223185 46.883185) (end 100.762 46.66) (stroke (width 0.15) (type solid)) (layer "Edge.Cuts"))
 (segment (start 146.92 93.5) (end 147 93.5) (width 0.25) (layer "F.Cu") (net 6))
 (segment (start 140.64 96.257919) (end 140.64 97.46) (width 0.5) (layer "F.Cu") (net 6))
 (segment (start 147 93.5) (end 147 93.64) (width 0.25) (layer "F.Cu") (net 6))
 (segment (start 137.982081 93.6) (end 140.64 96.257919) (width 0.5) (layer "F.Cu") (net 6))
 (segment (start 105.4 93.6) (end 137.982081 93.6) (width 0.5) (layer "F.Cu") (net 6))
 (segment (start 144.6 93.5) (end 140.64 97.46) (width 0.5) (layer "F.Cu") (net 6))
 (segment (start 146.92 93.5) (end 144.6 93.5) (width 0.5) (layer "F.Cu") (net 6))
 (segment (start 149.2 95.2) (end 149.2 93.76) (width 0.5) (layer "F.Cu") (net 5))
 (segment (start 147.379874 99.4) (end 148.291469 98.488405) (width 0.5) (layer "F.Cu") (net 5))
 (segment (start 138.1 97.46) (end 138.04 97.46) (width 0.25) (layer "F.Cu") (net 5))
 (segment (start 148.291469 96.108531) (end 149.2 95.2) (width 0.5) (layer "F.Cu") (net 5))
 (segment (start 138.04 97.46) (end 138 97.5) (width 0.25) (layer "F.Cu") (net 5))
 (segment (start 140.04 99.4) (end 147.379874 99.4) (width 0.5) (layer "F.Cu") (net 5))
 (segment (start 148.291469 98.488405) (end 148.291469 96.108531) (width 0.5) (layer "F.Cu") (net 5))
 (segment (start 138.1 97.46) (end 140.04 99.4) (width 0.5) (layer "F.Cu") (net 5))
 (segment (start 149.2 93.76) (end 149.46 93.5) (width 0.5) (layer "F.Cu") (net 5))
 (segment (start 150.8 97.46) (end 150.8 95.61) (width 0.5) (layer "F.Cu") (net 8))
 (segment (start 150.8 95.61) (end 152 94.41) (width 0.5) (layer "F.Cu") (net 8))
 (segment (start 152 94.41) (end 152 93.5) (width 0.5) (layer "F.Cu") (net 8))
 (segment (start 128.956 49.644) (end 128.956 49.2) (width 0.5) (layer "F.Cu") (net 15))
 (segment (start 114.6 66.52) (end 114.6 64) (width 0.5) (layer "F.Cu") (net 15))
 (segment (start 114.6 64) (end 128.956 49.644) (width 0.5) (layer "F.Cu") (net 15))
 (segment (start 131.496 50.096) (end 131.496 49.2) (width 0.5) (layer "F.Cu") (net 16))
 (segment (start 120.4 61.4) (end 131.6 50.2) (width 0.5) (layer "F.Cu") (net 16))
 (segment (start 142.2 89.6) (end 121.4 89.6) (width 0.5) (layer "F.Cu") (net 16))
 (segment (start 146.36 85.44) (end 142.2 89.6) (width 0.5) (layer "F.Cu") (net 16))
 (segment (start 146.36 79.64) (end 146.36 85.44) (width 0.5) (layer "F.Cu") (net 16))
 (segment (start 131.6 50.2) (end 131.496 50.096) (width 0.5) (layer "F.Cu") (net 16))
 (segment (start 121.4 89.6) (end 120.4 88.6) (width 0.5) (layer "F.Cu") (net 16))
 (segment (start 120.4 88.6) (end 120.4 61.4) (width 0.5) (layer "F.Cu") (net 16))
 (segment (start 132.8 59.8) (end 140.4 52.2) (width 0.5) (layer "F.Cu") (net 20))
 (segment (start 141.656 50.744) (end 141.656 49.2) (width 0.5) (layer "F.Cu") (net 20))
 (segment (start 140.4 52.2) (end 140.4 52) (width 0.5) (layer "F.Cu") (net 20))
 (segment (start 132.8 65.6) (end 132.8 59.8) (width 0.5) (layer "F.Cu") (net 20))
 (segment (start 140.4 52) (end 141.656 50.744) (width 0.5) (layer "F.Cu") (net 20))
 (segment (start 136.04 79.64) (end 136.2 79.64) (width 1) (layer "F.Cu") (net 20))
 (segment (start 136.2 69) (end 132.8 65.6) (width 0.5) (layer "F.Cu") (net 20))
 (segment (start 136.04 79.64) (end 136 79.6) (width 1) (layer "F.Cu") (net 20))
 (segment (start 136.2 79.64) (end 136.2 69) (width 0.5) (layer "F.Cu") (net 20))
 (segment (start 142.592103 53.607898) (end 142.592103 52.327897) (width 0.5) (layer "F.Cu") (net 21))
 (segment (start 142.592103 52.327897) (end 145.72 49.2) (width 0.5) (layer "F.Cu") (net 21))
 (segment (start 143.82 83.78) (end 139.8 87.8) (width 0.5) (layer "F.Cu") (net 17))
 (segment (start 143.82 79.64) (end 143.82 83.78) (width 0.5) (layer "F.Cu") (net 17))
 (segment (start 139.8 87.8) (end 123.6 87.8) (width 0.5) (layer "F.Cu") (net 17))
 (segment (start 123.6 60.8) (end 134.036 50.364) (width 0.5) (layer "F.Cu") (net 17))
 (segment (start 134.036 50.364) (end 134.036 49.2) (width 0.5) (layer "F.Cu") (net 17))
 (segment (start 123.6 87.8) (end 123.6 60.8) (width 0.5) (layer "F.Cu") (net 17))
 (segment (start 136.576 50.424) (end 136.576 49.2) (width 0.5) (layer "F.Cu") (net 18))
 (segment (start 141.28 79.64) (end 141.28 82.32) (width 0.5) (layer "F.Cu") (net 18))
 (segment (start 141.28 82.32) (end 137.8 85.8) (width 0.5) (layer "F.Cu") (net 18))
 (segment (start 130.6 85.8) (end 129.2 84.4) (width 0.5) (layer "F.Cu") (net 18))
 (segment (start 129.2 84.4) (end 129.2 57.8) (width 0.5) (layer "F.Cu") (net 18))
 (segment (start 129.2 57.8) (end 136.576 50.424) (width 0.5) (layer "F.Cu") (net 18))
 (segment (start 137.8 85.8) (end 130.6 85.8) (width 0.5) (layer "F.Cu") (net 18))
 (segment (start 131 59) (end 139.116 50.884) (width 0.5) (layer "F.Cu") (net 19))
 (segment (start 138.74 79.64) (end 138.74 81.66) (width 0.5) (layer "F.Cu") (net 19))
 (segment (start 133 83.2) (end 132.8 83) (width 0.5) (layer "F.Cu") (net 19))
 (segment (start 137.2 83.2) (end 133 83.2) (width 0.5) (layer "F.Cu") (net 19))
 (segment (start 132.8 71) (end 131 69.2) (width 0.5) (layer "F.Cu") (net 19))
 (segment (start 139.116 50.884) (end 139.116 49.2) (width 0.5) (layer "F.Cu") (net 19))
 (segment (start 138.74 81.66) (end 137.2 83.2) (width 0.5) (layer "F.Cu") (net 19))
 (segment (start 132.8 83) (end 132.8 71) (width 0.5) (layer "F.Cu") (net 19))
 (segment (start 131 69.2) (end 131 59) (width 0.5) (layer "F.Cu") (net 19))
 (segment (start 154.392103 52.807898) (end 153.34 51.755795) (width 0.5) (layer "F.Cu") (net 24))
 (segment (start 153.34 51.755795) (end 153.34 49.2) (width 0.5) (layer "F.Cu") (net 24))
 (segment (start 148.9 64.4) (end 165 64.4) (width 0.5) (layer "F.Cu") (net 26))
 (segment (start 165.4 60.2) (end 165.4 57.2) (width 0.5) (layer "F.Cu") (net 26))
 (segment (start 165 64.4) (end 167.3 62.1) (width 0.5) (layer "F.Cu") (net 26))
 (segment (start 165.4 57.2) (end 158.42 50.22) (width 0.5) (layer "F.Cu") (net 26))
 (segment (start 158.42 50.22) (end 158.42 49.2) (width 0.5) (layer "F.Cu") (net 26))
 (segment (start 167.3 62.1) (end 165.4 60.2) (width 0.5) (layer "F.Cu") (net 26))
 (segment (start 142.6 57.07868) (end 148.26 51.41868) (width 0.5) (layer "F.Cu") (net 22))
 (segment (start 138.74 63.26) (end 142.6 59.4) (width 0.5) (layer "F.Cu") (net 22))
 (segment (start 142.6 59.4) (end 142.6 57.07868) (width 0.5) (layer "F.Cu") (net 22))
 (segment (start 138.74 64.4) (end 138.74 63.26) (width 0.5) (layer "F.Cu") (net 22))
 (segment (start 148.26 51.41868) (end 148.26 49.2) (width 0.5) (layer "F.Cu") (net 22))
 (segment (start 150.8 51.8) (end 150.8 49.2) (width 0.5) (layer "F.Cu") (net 23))
 (segment (start 144.6 60) (end 144.6 58) (width 0.5) (layer "F.Cu") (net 23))
 (segment (start 141.28 64.4) (end 141.28 63.32) (width 0.5) (layer "F.Cu") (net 23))
 (segment (start 141.28 63.32) (end 144.6 60) (width 0.5) (layer "F.Cu") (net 23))
 (segment (start 141.28 64.4) (end 141.4 64.4) (width 1) (layer "F.Cu") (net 23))
 (segment (start 144.6 58) (end 150.8 51.8) (width 0.5) (layer "F.Cu") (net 23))
 (segment (start 155.88 50.68) (end 155.88 49.2) (width 0.5) (layer "F.Cu") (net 25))
 (segment (start 163.2 60.6) (end 163.2 58) (width 0.5) (layer "F.Cu") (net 25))
 (segment (start 163.2 58) (end 155.88 50.68) (width 0.5) (layer "F.Cu") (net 25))
 (segment (start 145.54 97.46) (end 145.5 97.5) (width 0.25) (layer "F.Cu") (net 7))
 (segment (start 145.72 97.46) (end 145.54 97.46) (width 0.25) (layer "F.Cu") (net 7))
 (segment (start 136.2 64.4) (end 136.2 61.584205) (width 0.5) (layer "F.Cu") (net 29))
 (segment (start 102.2 49.05) (end 102.25 49.05) (width 0.25) (layer "F.Cu") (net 29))
 (segment (start 136.2 61.584205) (end 135.407898 60.792103) (width 0.5) (layer "F.Cu") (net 29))
 (segment (start 146.36 64.4) (end 146.36 64.56) (width 0.5) (layer "F.Cu") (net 33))
 (segment (start 150.225126 60.6) (end 153.04 60.6) (width 0.5) (layer "F.Cu") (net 33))
 (segment (start 146.4 64.425126) (end 150.225126 60.6) (width 0.5) (layer "F.Cu") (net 33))
 (segment (start 146.36 64.56) (end 146.4 64.6) (width 0.5) (layer "F.Cu") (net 33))
 (segment (start 146.4 64.6) (end 146.4 64.425126) (width 0.5) (layer "F.Cu") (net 33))
 (segment (start 147.207898 61.012102) (end 147.207898 59.992103) (width 0.5) (layer "F.Cu") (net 34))
 (segment (start 143.82 64.4) (end 147.207898 61.012102) (width 0.5) (layer "F.Cu") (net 34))
 (segment (start 143 91.6) (end 148 86.6) (width 0.5) (layer "F.Cu") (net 32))
 (segment (start 118 89) (end 120.6 91.6) (width 0.5) (layer "F.Cu") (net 32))
 (segment (start 148.2 86.6) (end 148.9 85.9) (width 0.5) (layer "F.Cu") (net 32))
 (segment (start 148.9 85.9) (end 148.9 79.64) (width 0.5) (layer "F.Cu") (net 32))
 (segment (start 114.6 76.68) (end 118 80.08) (width 0.5) (layer "F.Cu") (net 32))
 (segment (start 118 80.08) (end 118 89) (width 0.5) (layer "F.Cu") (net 32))
 (segment (start 120.6 91.6) (end 143 91.6) (width 0.5) (layer "F.Cu") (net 32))
 (segment (start 148 86.6) (end 148.2 86.6) (width 0.5) (layer "F.Cu") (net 32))
 (segment (start 107.7 89.1) (end 101.9 89.1) (width 0.5) (layer "F.Cu") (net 31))
 (segment (start 110 91.4) (end 107.7 89.1) (width 0.5) (layer "F.Cu") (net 31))
 (segment (start 116.4 91.4) (end 110 91.4) (width 0.5) (layer "F.Cu") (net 31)))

